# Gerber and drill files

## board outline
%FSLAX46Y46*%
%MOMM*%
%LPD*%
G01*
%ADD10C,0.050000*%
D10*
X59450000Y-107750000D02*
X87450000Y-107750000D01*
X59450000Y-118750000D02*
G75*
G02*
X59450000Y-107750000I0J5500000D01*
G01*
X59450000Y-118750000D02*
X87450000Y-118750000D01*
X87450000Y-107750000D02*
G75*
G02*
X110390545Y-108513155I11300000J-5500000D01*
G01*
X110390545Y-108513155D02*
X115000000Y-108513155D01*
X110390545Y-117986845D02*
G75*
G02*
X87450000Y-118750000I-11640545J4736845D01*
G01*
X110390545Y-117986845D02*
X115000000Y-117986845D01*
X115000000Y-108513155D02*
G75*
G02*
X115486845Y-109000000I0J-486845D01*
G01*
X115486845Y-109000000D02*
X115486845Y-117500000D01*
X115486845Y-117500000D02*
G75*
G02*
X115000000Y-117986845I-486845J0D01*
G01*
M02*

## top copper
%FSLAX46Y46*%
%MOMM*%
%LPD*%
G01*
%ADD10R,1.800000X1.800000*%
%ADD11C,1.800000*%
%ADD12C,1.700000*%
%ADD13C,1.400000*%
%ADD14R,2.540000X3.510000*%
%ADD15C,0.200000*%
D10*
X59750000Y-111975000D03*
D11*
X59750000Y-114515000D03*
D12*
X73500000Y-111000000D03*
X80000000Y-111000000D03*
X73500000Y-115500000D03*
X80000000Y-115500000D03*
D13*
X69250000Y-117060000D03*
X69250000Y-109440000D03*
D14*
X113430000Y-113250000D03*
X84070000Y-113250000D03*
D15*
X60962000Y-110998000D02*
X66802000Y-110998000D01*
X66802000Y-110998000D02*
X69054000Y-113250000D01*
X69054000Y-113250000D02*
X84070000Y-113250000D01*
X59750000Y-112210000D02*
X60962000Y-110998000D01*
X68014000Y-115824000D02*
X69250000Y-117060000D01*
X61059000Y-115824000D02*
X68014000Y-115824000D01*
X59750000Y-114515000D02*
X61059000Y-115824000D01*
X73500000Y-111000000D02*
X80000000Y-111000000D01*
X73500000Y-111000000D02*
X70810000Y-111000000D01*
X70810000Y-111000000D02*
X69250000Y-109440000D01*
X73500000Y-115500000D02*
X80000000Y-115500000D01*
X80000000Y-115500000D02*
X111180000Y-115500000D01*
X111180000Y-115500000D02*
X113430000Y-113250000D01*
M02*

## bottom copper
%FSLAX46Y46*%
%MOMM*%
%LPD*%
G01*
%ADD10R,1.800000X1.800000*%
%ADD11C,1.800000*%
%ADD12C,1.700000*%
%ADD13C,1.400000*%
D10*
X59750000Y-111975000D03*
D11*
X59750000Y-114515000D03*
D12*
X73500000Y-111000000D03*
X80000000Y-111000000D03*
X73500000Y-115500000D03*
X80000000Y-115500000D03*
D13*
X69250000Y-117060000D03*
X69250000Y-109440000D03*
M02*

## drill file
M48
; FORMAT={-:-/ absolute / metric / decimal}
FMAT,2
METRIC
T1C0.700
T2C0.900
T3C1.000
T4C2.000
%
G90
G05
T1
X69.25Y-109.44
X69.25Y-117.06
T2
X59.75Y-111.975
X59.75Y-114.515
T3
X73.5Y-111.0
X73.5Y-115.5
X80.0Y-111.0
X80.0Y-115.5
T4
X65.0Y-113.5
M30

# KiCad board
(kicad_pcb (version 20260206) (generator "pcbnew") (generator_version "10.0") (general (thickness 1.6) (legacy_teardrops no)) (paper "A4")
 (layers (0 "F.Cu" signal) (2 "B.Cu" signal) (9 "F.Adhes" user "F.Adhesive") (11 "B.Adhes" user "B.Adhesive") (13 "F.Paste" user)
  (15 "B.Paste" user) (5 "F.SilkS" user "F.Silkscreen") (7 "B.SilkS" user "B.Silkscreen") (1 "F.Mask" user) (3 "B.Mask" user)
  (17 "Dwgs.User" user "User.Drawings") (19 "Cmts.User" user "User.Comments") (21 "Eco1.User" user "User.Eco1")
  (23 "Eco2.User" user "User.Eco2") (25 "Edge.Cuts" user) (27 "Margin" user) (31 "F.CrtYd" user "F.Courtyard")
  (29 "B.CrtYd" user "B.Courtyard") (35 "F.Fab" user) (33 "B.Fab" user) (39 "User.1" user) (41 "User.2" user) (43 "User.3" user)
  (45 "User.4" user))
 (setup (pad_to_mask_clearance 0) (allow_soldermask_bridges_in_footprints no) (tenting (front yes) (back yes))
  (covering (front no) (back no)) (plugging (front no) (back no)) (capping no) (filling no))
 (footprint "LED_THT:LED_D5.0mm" (layer "F.Cu") (at 59.75 111.975 -90)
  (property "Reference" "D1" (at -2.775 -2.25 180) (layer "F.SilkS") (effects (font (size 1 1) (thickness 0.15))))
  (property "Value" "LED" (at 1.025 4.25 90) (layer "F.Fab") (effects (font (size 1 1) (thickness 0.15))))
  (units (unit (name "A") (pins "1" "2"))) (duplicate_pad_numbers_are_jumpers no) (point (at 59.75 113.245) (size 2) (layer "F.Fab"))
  (pad "1" thru_hole rect (at 0 0 270) (size 1.8 1.8) (drill 0.9) (layers "*.Cu" "*.Mask") (remove_unused_layers no) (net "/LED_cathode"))
  (pad "2" thru_hole circle (at 2.54 0 270) (size 1.8 1.8) (drill 0.9) (layers "*.Cu" "*.Mask") (remove_unused_layers no) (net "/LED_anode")))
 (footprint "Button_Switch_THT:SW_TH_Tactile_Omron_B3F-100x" (layer "F.Cu") (at 73.5 111)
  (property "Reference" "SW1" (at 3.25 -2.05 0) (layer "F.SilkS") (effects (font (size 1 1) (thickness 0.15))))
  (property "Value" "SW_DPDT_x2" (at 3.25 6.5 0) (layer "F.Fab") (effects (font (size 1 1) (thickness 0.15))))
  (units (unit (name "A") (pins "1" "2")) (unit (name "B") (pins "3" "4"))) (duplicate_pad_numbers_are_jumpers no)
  (pad "1" thru_hole circle (at 0 0) (size 1.7 1.7) (drill 1) (layers "*.Cu" "*.Mask") (remove_unused_layers no) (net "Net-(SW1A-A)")
   (thermal_bridge_angle 90))
  (pad "1" thru_hole circle (at 6.5 0) (size 1.7 1.7) (drill 1) (layers "*.Cu" "*.Mask") (remove_unused_layers no) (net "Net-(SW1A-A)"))
  (pad "2" thru_hole circle (at 0 4.5) (size 1.7 1.7) (drill 1) (layers "*.Cu" "*.Mask") (remove_unused_layers no) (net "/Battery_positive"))
  (pad "2" thru_hole circle (at 6.5 4.5) (size 1.7 1.7) (drill 1) (layers "*.Cu" "*.Mask") (remove_unused_layers no)
   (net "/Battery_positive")))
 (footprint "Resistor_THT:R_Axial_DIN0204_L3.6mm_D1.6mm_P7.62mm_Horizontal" (layer "F.Cu") (at 69.25 117.06 90)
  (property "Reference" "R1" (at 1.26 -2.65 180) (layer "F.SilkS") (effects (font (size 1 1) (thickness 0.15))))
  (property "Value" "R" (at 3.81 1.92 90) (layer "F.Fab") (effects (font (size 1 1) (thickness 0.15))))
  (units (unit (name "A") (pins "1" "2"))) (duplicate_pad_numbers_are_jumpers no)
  (pad "1" thru_hole circle (at 0 0 90) (size 1.4 1.4) (drill 0.7) (layers "*.Cu" "*.Mask") (remove_unused_layers no) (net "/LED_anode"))
  (pad "2" thru_hole circle (at 7.62 0 90) (size 1.4 1.4) (drill 0.7) (layers "*.Cu" "*.Mask") (remove_unused_layers no)
   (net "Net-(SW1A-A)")))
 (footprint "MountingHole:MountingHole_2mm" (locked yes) (layer "F.Cu") (at 65 113.5)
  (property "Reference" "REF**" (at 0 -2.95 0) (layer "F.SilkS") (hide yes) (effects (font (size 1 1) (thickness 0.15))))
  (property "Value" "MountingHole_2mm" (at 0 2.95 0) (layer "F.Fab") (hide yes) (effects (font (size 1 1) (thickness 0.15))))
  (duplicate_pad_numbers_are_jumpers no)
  (pad "" np_thru_hole circle (at 0 0) (size 2 2) (drill 2) (layers "*.Cu" "*.Mask")))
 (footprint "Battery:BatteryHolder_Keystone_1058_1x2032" (layer "F.Cu") (at 98.75 113.25 180)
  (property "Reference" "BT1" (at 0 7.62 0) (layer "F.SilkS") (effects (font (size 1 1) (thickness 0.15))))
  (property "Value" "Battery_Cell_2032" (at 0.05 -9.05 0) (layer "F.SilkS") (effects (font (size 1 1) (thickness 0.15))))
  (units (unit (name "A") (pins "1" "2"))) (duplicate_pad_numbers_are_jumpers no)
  (pad "1" smd rect (at -14.68 0 180) (size 2.54 3.51) (layers "F.Cu" "F.Mask" "F.Paste") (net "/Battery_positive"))
  (pad "2" smd rect (at 14.68 0 180) (size 2.54 3.51) (layers "F.Cu" "F.Mask" "F.Paste") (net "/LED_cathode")))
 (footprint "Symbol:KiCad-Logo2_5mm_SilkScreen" (layer "B.Cu") (at 98.5 109 180)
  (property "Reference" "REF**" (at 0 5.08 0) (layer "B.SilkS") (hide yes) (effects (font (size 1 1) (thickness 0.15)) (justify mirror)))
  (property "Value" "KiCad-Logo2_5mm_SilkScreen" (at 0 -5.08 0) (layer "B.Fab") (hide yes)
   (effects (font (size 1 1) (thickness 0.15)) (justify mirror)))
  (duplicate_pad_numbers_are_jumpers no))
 (gr_line (start 59.45 107.75) (end 87.45 107.75) (stroke (width 0.05) (type default)) (locked yes) (layer "Edge.Cuts"))
 (gr_arc (start 59.45 118.75) (mid 53.95 113.25) (end 59.45 107.75) (stroke (width 0.05) (type default)) (locked yes) (layer "Edge.Cuts"))
 (gr_line (start 59.45 118.75) (end 87.45 118.75) (stroke (width 0.05) (type default)) (locked yes) (layer "Edge.Cuts"))
 (gr_arc (start 87.45 107.75) (mid 99.167845 100.68953) (end 110.390545 108.513155) (stroke (width 0.05) (type default)) (locked yes)
  (layer "Edge.Cuts"))
 (gr_line (start 110.390545 108.513155) (end 115 108.513155) (stroke (width 0.05) (type default)) (locked yes) (layer "Edge.Cuts"))
 (gr_arc (start 110.390545 117.986845) (mid 99.167845 125.81047) (end 87.45 118.75) (stroke (width 0.05) (type default)) (locked yes)
  (layer "Edge.Cuts"))
 (gr_line (start 110.390545 117.986845) (end 115 117.986845) (stroke (width 0.05) (type default)) (locked yes) (layer "Edge.Cuts"))
 (gr_arc (start 115 108.513155) (mid 115.344251 108.655749) (end 115.486845 109) (stroke (width 0.05) (type default)) (locked yes)
  (layer "Edge.Cuts"))
 (gr_line (start 115.486845 109) (end 115.486845 117.5) (stroke (width 0.05) (type default)) (locked yes) (layer "Edge.Cuts"))
 (gr_arc (start 115.486845 117.5) (mid 115.344251 117.844251) (end 115 117.986845) (stroke (width 0.05) (type default)) (locked yes)
  (layer "Edge.Cuts"))
 (segment (start 60.962 110.998) (end 66.802 110.998) (width 0.2) (layer "F.Cu") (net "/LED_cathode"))
 (segment (start 66.802 110.998) (end 69.054 113.25) (width 0.2) (layer "F.Cu") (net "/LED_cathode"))
 (segment (start 69.054 113.25) (end 84.07 113.25) (width 0.2) (layer "F.Cu") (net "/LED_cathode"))
 (segment (start 59.75 112.21) (end 60.962 110.998) (width 0.2) (layer "F.Cu") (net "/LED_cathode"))
 (segment (start 68.014 115.824) (end 69.25 117.06) (width 0.2) (layer "F.Cu") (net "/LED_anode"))
 (segment (start 61.059 115.824) (end 68.014 115.824) (width 0.2) (layer "F.Cu") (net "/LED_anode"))
 (segment (start 59.75 114.515) (end 61.059 115.824) (width 0.2) (layer "F.Cu") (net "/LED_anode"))
 (segment (start 73.5 111) (end 80 111) (width 0.2) (layer "F.Cu") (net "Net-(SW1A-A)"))
 (segment (start 73.5 111) (end 70.81 111) (width 0.2) (layer "F.Cu") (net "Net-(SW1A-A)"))
 (segment (start 70.81 111) (end 69.25 109.44) (width 0.2) (layer "F.Cu") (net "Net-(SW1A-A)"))
 (segment (start 73.5 115.5) (end 80 115.5) (width 0.2) (layer "F.Cu") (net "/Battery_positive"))
 (segment (start 80 115.5) (end 111.18 115.5) (width 0.2) (layer "F.Cu") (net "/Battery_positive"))
 (segment (start 111.18 115.5) (end 113.43 113.25) (width 0.2) (layer "F.Cu") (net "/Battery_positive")))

